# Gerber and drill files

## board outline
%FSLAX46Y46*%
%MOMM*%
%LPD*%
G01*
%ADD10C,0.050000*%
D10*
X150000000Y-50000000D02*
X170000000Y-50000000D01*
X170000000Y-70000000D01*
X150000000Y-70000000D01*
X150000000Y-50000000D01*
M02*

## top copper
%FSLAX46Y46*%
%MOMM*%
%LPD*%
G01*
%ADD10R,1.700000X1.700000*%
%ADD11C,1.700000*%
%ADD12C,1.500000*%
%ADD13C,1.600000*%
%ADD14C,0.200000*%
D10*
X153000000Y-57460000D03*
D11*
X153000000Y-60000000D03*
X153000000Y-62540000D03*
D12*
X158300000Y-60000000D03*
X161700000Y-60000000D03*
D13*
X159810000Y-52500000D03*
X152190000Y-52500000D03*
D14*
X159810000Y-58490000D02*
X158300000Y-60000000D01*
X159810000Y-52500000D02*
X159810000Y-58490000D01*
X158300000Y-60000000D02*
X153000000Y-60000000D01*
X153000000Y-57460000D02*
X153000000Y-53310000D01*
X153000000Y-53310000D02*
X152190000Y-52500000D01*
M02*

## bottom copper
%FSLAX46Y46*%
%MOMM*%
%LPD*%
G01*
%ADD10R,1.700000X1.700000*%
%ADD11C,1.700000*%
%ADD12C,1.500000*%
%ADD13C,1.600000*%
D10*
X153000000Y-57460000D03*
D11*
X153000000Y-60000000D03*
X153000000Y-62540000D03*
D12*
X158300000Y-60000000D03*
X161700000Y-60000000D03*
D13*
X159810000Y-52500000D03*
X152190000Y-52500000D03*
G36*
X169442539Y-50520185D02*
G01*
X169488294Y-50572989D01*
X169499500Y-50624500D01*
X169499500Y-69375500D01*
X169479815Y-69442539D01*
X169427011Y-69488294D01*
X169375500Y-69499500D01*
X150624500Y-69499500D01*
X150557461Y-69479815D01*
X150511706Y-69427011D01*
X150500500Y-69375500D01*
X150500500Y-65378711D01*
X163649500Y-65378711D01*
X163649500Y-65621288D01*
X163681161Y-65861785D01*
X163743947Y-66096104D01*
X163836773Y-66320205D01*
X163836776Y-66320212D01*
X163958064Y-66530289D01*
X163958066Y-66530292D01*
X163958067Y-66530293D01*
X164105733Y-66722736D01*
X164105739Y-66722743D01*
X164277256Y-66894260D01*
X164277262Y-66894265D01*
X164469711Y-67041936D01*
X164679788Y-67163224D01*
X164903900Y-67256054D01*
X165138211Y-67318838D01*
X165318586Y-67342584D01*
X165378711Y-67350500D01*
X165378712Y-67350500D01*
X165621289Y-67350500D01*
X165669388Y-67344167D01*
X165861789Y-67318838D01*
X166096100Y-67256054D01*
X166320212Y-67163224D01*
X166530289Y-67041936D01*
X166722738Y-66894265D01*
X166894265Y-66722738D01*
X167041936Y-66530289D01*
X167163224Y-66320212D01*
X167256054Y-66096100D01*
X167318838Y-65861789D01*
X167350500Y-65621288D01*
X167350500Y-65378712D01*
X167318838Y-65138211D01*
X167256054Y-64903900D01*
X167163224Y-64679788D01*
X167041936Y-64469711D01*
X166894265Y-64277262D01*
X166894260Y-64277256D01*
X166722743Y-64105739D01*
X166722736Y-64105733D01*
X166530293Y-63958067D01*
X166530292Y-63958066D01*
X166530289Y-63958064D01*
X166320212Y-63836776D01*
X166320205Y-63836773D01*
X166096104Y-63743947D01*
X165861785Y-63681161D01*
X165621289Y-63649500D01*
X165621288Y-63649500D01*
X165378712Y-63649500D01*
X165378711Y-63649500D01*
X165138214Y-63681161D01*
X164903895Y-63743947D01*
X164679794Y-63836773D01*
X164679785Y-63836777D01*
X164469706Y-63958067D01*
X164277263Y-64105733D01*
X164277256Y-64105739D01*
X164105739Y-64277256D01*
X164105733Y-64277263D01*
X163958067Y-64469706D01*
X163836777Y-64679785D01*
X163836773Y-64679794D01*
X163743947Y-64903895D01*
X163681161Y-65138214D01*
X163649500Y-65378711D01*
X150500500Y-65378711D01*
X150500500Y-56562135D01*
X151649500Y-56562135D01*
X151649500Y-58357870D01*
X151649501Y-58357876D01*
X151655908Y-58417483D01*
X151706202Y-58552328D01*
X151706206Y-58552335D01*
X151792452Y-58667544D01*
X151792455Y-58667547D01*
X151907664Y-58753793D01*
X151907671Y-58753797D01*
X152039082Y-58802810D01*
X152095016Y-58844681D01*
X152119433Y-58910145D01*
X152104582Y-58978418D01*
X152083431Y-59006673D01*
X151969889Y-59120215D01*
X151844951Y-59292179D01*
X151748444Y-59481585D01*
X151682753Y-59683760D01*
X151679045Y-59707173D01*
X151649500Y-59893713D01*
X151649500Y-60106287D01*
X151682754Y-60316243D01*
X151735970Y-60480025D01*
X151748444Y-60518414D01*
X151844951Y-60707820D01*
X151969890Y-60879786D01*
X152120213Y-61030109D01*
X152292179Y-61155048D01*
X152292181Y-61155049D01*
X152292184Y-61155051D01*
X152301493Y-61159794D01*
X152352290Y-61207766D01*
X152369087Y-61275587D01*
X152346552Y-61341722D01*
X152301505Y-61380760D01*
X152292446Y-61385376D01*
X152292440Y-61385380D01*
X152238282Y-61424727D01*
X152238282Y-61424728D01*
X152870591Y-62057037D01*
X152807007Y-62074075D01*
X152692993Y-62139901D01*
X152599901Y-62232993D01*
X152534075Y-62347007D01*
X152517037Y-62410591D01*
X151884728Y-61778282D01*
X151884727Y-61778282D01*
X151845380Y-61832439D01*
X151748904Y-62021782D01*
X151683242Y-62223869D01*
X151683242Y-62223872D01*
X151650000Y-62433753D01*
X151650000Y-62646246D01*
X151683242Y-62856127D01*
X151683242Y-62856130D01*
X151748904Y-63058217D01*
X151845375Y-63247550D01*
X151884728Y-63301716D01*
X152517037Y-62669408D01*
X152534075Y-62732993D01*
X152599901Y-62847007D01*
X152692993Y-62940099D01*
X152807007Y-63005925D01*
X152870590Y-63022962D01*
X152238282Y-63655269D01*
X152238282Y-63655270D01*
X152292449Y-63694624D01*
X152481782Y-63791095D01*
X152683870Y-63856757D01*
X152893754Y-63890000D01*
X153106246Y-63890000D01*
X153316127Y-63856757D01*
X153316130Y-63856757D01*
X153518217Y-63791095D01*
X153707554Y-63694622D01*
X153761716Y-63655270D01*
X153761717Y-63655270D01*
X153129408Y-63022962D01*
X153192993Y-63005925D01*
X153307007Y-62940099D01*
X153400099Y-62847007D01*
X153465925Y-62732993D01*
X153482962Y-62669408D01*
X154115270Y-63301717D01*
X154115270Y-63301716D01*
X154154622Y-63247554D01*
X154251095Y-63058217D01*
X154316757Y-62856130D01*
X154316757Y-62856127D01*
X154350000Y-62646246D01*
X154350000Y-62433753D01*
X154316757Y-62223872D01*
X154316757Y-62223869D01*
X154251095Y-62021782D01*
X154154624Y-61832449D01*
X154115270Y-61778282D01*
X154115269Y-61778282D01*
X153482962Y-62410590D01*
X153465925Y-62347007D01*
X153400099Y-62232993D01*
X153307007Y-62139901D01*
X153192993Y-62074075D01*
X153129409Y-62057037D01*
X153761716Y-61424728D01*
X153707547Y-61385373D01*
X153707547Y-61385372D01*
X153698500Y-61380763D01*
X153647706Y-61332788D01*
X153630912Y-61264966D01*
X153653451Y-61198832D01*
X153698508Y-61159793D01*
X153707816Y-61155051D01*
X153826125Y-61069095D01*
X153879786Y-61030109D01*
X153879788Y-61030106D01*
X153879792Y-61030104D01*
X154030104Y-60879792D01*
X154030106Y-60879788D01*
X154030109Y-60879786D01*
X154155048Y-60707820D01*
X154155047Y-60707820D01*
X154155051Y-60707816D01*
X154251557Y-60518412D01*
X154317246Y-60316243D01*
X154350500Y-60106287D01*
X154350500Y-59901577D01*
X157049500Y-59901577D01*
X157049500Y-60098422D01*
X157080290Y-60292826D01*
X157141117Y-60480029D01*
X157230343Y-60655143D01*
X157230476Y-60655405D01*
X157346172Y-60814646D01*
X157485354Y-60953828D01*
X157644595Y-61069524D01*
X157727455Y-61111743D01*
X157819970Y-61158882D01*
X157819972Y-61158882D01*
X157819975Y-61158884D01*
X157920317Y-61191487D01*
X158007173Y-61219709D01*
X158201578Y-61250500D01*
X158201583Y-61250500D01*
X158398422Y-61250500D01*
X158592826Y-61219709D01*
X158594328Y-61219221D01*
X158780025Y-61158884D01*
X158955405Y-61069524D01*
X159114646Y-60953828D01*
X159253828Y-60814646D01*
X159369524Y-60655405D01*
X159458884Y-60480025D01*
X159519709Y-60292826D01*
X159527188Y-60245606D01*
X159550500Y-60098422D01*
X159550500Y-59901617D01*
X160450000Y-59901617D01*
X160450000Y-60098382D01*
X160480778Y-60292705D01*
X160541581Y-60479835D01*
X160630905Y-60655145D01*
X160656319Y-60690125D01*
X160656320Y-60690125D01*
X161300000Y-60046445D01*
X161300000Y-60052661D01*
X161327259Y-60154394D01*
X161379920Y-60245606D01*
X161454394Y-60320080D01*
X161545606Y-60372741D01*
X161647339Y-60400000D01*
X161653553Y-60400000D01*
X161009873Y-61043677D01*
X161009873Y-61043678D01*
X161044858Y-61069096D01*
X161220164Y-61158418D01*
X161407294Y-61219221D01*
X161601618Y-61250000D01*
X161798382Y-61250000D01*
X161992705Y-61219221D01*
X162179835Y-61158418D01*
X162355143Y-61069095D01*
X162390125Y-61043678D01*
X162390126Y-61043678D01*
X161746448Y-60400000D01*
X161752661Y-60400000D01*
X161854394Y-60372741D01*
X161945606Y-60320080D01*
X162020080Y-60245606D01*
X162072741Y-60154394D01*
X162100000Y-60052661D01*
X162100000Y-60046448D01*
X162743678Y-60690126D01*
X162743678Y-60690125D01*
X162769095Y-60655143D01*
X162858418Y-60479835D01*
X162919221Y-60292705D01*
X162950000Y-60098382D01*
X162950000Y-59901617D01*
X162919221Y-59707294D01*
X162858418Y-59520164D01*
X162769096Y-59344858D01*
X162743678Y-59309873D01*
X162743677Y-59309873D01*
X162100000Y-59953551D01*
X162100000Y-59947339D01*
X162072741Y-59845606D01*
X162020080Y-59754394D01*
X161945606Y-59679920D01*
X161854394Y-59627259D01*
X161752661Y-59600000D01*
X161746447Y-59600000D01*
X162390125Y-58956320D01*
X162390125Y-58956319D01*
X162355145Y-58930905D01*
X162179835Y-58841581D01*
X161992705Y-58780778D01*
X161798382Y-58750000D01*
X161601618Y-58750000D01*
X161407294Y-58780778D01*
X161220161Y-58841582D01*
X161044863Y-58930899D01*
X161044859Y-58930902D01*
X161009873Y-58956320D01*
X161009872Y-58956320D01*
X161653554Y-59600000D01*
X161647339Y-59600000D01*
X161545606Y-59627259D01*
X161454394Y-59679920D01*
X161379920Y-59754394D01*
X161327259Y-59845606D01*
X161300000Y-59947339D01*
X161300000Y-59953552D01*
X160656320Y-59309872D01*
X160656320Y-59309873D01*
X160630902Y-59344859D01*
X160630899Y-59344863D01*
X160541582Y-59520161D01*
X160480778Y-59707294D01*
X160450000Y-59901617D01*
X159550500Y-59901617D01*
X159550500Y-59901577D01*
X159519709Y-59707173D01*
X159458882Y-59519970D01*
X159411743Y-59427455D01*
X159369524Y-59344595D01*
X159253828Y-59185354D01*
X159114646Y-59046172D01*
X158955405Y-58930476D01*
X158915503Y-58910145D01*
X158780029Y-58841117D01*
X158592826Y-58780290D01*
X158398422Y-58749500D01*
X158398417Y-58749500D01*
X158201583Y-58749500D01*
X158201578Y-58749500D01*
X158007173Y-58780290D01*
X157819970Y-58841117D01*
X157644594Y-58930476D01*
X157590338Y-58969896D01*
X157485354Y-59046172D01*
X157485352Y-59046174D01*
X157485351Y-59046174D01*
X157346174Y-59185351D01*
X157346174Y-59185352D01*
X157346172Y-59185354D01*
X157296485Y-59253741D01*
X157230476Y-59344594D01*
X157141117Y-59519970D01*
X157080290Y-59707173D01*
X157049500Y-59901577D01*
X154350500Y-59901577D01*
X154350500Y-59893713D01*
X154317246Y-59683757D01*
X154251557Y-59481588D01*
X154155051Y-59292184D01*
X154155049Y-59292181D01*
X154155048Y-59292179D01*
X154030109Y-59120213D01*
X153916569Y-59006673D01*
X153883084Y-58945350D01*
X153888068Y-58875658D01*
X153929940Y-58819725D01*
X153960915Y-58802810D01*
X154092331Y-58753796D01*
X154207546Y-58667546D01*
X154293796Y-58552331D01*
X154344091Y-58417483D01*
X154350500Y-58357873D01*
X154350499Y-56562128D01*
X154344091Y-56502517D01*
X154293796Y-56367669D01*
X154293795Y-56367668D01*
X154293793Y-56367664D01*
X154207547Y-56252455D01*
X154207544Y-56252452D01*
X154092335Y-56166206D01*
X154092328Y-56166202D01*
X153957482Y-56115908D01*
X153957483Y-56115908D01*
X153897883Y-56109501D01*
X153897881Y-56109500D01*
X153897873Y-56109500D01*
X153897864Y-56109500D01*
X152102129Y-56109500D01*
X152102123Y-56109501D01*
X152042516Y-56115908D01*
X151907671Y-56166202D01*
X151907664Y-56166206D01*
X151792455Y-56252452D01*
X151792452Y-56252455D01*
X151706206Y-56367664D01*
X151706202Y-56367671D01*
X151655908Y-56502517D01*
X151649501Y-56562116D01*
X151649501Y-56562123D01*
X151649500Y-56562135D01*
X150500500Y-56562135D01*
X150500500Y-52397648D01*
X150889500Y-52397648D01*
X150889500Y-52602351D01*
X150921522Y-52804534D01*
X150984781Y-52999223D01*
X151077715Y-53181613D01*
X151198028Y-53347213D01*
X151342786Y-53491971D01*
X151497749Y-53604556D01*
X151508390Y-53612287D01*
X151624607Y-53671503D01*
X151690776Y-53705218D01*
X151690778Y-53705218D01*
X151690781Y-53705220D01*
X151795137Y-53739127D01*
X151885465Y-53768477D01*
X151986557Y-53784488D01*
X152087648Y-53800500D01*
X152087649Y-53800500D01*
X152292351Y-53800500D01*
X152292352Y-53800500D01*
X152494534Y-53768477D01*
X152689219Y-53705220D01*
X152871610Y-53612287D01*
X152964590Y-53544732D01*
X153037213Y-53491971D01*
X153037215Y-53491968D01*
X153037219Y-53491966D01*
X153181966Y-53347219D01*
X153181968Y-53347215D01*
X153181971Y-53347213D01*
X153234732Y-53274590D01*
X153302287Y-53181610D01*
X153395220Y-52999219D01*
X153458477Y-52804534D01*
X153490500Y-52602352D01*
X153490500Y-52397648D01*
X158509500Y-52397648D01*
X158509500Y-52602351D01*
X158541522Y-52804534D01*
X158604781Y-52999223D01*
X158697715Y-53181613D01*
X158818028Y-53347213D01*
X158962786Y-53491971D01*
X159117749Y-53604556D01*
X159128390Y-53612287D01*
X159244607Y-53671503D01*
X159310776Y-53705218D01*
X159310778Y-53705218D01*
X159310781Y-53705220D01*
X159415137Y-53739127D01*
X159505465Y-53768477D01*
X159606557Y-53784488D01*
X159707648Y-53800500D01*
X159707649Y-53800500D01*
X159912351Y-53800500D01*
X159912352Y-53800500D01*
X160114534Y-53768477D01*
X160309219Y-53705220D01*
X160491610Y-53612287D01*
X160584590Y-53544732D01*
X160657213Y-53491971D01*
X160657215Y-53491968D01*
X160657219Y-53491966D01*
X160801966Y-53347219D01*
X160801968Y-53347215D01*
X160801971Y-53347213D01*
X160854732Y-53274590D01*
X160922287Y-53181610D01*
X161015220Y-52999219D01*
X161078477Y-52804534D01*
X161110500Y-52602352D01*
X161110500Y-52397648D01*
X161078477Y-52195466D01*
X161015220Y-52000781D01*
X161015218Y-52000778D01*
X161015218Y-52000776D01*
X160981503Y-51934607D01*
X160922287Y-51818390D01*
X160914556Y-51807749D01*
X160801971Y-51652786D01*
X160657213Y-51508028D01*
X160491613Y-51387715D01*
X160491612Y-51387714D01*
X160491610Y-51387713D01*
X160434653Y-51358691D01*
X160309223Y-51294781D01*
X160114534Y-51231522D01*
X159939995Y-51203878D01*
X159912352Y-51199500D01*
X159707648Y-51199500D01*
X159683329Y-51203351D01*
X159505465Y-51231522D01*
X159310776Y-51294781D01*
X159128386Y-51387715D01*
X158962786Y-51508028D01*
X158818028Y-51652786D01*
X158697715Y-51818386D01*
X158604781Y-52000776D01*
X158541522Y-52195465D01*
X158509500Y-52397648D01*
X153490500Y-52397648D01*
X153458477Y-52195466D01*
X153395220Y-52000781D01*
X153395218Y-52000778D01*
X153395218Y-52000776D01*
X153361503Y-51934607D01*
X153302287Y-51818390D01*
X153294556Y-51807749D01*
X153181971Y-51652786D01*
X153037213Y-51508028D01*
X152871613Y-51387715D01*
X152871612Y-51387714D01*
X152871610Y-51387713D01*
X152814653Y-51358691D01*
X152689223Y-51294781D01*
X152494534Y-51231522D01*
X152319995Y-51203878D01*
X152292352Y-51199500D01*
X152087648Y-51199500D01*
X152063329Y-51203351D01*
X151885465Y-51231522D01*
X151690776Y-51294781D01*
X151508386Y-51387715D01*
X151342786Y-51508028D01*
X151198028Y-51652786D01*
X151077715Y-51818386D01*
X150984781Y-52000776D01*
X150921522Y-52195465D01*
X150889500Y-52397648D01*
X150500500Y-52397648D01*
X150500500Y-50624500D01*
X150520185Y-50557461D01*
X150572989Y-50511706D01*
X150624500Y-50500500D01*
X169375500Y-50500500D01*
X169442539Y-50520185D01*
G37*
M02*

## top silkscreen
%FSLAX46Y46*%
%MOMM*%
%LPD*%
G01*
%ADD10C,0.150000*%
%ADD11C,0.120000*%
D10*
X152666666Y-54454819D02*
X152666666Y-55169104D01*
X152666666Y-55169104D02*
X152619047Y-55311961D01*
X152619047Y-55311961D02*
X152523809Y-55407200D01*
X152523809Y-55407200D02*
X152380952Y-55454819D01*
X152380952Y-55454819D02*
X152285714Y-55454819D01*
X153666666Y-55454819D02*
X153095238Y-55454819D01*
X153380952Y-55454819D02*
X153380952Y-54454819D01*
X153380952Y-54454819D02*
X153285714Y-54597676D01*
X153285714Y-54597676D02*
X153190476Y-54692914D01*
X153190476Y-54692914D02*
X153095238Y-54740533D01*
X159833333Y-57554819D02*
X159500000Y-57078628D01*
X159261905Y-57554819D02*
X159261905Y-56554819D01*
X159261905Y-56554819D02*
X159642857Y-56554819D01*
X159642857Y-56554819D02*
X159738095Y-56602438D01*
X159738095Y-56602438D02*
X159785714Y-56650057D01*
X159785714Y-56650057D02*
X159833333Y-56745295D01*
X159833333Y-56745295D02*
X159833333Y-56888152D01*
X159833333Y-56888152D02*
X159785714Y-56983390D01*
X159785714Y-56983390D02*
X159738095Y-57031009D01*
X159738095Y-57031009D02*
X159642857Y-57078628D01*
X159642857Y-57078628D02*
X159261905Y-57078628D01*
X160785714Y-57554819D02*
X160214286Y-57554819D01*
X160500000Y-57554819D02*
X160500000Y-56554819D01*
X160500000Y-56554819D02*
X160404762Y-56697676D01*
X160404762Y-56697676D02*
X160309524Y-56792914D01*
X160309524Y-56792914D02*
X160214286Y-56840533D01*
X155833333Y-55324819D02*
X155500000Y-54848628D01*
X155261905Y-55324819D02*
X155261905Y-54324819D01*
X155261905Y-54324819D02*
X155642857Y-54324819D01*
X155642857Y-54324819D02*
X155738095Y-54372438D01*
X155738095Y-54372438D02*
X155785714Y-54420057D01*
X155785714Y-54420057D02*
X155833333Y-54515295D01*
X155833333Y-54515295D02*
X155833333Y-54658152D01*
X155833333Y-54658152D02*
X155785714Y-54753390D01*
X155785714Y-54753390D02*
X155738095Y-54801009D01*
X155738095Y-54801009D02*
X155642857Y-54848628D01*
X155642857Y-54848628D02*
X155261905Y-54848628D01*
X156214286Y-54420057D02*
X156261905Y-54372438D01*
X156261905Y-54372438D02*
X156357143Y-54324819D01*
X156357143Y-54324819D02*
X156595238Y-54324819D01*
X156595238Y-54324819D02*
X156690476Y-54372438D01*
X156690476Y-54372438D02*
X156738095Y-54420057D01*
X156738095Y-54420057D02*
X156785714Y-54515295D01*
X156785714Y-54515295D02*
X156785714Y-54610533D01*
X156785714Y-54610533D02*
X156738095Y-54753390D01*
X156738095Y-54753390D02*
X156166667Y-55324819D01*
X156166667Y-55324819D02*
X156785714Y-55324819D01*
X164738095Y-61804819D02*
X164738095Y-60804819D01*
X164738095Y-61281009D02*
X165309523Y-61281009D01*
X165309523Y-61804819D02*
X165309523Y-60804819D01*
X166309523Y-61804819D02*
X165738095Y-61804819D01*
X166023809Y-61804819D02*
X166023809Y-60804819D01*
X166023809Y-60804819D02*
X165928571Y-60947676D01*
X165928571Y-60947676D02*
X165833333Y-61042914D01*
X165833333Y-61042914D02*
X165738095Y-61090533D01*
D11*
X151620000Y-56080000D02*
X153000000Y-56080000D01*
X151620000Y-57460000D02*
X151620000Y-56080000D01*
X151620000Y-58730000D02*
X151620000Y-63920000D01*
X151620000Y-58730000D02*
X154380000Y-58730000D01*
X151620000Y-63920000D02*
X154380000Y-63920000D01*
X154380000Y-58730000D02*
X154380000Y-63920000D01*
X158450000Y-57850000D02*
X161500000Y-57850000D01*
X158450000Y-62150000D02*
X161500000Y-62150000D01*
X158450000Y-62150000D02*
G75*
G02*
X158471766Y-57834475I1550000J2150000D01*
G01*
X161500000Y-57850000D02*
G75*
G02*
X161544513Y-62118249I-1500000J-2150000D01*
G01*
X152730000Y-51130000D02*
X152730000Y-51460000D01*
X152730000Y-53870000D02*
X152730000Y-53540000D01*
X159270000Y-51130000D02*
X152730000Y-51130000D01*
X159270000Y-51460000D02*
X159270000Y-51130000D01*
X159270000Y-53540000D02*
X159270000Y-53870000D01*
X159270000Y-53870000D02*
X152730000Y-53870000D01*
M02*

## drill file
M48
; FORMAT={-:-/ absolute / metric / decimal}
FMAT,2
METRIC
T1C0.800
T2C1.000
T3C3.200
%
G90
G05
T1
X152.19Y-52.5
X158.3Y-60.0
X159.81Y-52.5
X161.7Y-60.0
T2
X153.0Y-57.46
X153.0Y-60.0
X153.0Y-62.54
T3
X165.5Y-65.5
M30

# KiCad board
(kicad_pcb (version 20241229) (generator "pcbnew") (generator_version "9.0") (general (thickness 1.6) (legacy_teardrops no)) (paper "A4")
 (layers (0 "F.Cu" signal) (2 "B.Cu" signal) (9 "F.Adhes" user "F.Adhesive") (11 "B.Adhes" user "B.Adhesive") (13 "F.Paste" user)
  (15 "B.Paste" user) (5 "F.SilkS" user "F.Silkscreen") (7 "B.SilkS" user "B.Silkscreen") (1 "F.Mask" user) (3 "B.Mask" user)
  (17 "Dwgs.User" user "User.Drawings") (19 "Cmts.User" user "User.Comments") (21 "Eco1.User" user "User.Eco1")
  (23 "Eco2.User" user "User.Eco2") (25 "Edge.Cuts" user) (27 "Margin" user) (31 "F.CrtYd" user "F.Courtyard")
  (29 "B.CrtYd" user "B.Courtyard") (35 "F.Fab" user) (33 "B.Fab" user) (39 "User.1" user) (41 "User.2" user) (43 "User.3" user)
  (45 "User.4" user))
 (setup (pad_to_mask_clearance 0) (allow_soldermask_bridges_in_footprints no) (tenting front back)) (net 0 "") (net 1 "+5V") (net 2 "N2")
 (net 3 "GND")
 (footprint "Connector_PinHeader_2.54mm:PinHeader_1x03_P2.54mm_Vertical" (layer "F.Cu") (at 153 57.46)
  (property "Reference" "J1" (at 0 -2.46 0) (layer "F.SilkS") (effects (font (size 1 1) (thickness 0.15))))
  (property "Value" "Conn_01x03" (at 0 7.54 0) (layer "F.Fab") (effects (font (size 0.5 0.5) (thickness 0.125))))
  (fp_line (start -1.38 -1.38) (end 0 -1.38) (stroke (width 0.12) (type solid)) (layer "F.SilkS"))
  (fp_line (start -1.38 0) (end -1.38 -1.38) (stroke (width 0.12) (type solid)) (layer "F.SilkS"))
  (fp_line (start -1.38 1.27) (end -1.38 6.46) (stroke (width 0.12) (type solid)) (layer "F.SilkS"))
  (fp_line (start -1.38 1.27) (end 1.38 1.27) (stroke (width 0.12) (type solid)) (layer "F.SilkS"))
  (fp_line (start -1.38 6.46) (end 1.38 6.46) (stroke (width 0.12) (type solid)) (layer "F.SilkS"))
  (fp_line (start 1.38 1.27) (end 1.38 6.46) (stroke (width 0.12) (type solid)) (layer "F.SilkS"))
  (pad "1" thru_hole rect (at 0 0) (size 1.7 1.7) (drill 1) (layers "*.Cu" "*.Mask") (remove_unused_layers no) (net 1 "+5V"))
  (pad "2" thru_hole circle (at 0 2.54) (size 1.7 1.7) (drill 1) (layers "*.Cu" "*.Mask") (remove_unused_layers no) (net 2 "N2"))
  (pad "3" thru_hole circle (at 0 5.08) (size 1.7 1.7) (drill 1) (layers "*.Cu" "*.Mask") (remove_unused_layers no) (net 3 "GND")))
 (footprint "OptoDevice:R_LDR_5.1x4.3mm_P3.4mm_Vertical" (layer "F.Cu") (at 158.3 60)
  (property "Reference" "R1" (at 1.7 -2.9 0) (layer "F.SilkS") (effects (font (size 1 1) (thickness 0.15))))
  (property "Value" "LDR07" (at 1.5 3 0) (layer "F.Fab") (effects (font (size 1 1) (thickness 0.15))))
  (fp_line (start 0.15 -2.15) (end 3.2 -2.15) (stroke (width 0.12) (type solid)) (layer "F.SilkS"))
  (fp_line (start 0.15 2.15) (end 3.2 2.15) (stroke (width 0.12) (type solid)) (layer "F.SilkS"))
  (fp_arc (start 0.15 2.15) (mid -0.950438 -0.013368) (end 0.171766 -2.165525) (stroke (width 0.12) (type solid)) (layer "F.SilkS"))
  (fp_arc (start 3.2 -2.15) (mid 4.321403 -0.027338) (end 3.244513 2.118249) (stroke (width 0.12) (type solid)) (layer "F.SilkS"))
  (pad "1" thru_hole circle (at 0 0) (size 1.5 1.5) (drill 0.8) (layers "*.Cu" "*.Mask") (remove_unused_layers no) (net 2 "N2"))
  (pad "2" thru_hole circle (at 3.4 0) (size 1.5 1.5) (drill 0.8) (layers "*.Cu" "*.Mask") (remove_unused_layers no) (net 3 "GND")))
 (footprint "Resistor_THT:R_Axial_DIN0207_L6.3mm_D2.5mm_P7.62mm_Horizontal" (layer "F.Cu") (at 159.81 52.5 180)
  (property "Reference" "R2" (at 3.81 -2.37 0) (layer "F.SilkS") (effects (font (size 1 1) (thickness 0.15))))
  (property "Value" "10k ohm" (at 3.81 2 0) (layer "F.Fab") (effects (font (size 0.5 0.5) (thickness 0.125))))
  (fp_line (start 7.08 1.37) (end 7.08 1.04) (stroke (width 0.12) (type solid)) (layer "F.SilkS"))
  (fp_line (start 7.08 -1.37) (end 7.08 -1.04) (stroke (width 0.12) (type solid)) (layer "F.SilkS"))
  (fp_line (start 0.54 1.37) (end 7.08 1.37) (stroke (width 0.12) (type solid)) (layer "F.SilkS"))
  (fp_line (start 0.54 1.04) (end 0.54 1.37) (stroke (width 0.12) (type solid)) (layer "F.SilkS"))
  (fp_line (start 0.54 -1.04) (end 0.54 -1.37) (stroke (width 0.12) (type solid)) (layer "F.SilkS"))
  (fp_line (start 0.54 -1.37) (end 7.08 -1.37) (stroke (width 0.12) (type solid)) (layer "F.SilkS"))
  (pad "1" thru_hole circle (at 0 0 180) (size 1.6 1.6) (drill 0.8) (layers "*.Cu" "*.Mask") (remove_unused_layers no) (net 2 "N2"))
  (pad "2" thru_hole circle (at 7.62 0 180) (size 1.6 1.6) (drill 0.8) (layers "*.Cu" "*.Mask") (remove_unused_layers no) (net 1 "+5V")))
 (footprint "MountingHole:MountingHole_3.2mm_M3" (layer "F.Cu") (at 165.5 65.5)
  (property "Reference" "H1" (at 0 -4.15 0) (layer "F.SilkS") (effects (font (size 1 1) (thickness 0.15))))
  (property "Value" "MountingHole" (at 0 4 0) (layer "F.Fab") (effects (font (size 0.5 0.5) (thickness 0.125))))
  (pad "" np_thru_hole circle (at 0 0) (size 3.2 3.2) (drill 3.2) (layers "*.Cu" "*.Mask")))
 (gr_rect (start 150 50) (end 170 70) (stroke (width 0.05) (type default)) (fill no) (layer "Edge.Cuts"))
 (segment (start 159.81 58.49) (end 158.3 60) (width 0.2) (layer "F.Cu") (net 2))
 (segment (start 159.81 52.5) (end 159.81 58.49) (width 0.2) (layer "F.Cu") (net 2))
 (segment (start 158.3 60) (end 153 60) (width 0.2) (layer "F.Cu") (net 2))
 (segment (start 153 57.46) (end 153 53.31) (width 0.2) (layer "F.Cu") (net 1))
 (segment (start 153 53.31) (end 152.19 52.5) (width 0.2) (layer "F.Cu") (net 1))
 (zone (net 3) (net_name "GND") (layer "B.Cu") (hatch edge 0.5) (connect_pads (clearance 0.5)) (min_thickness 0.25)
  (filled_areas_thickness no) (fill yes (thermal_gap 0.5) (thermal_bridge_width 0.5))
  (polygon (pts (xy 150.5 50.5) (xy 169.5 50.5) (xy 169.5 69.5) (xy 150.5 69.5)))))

